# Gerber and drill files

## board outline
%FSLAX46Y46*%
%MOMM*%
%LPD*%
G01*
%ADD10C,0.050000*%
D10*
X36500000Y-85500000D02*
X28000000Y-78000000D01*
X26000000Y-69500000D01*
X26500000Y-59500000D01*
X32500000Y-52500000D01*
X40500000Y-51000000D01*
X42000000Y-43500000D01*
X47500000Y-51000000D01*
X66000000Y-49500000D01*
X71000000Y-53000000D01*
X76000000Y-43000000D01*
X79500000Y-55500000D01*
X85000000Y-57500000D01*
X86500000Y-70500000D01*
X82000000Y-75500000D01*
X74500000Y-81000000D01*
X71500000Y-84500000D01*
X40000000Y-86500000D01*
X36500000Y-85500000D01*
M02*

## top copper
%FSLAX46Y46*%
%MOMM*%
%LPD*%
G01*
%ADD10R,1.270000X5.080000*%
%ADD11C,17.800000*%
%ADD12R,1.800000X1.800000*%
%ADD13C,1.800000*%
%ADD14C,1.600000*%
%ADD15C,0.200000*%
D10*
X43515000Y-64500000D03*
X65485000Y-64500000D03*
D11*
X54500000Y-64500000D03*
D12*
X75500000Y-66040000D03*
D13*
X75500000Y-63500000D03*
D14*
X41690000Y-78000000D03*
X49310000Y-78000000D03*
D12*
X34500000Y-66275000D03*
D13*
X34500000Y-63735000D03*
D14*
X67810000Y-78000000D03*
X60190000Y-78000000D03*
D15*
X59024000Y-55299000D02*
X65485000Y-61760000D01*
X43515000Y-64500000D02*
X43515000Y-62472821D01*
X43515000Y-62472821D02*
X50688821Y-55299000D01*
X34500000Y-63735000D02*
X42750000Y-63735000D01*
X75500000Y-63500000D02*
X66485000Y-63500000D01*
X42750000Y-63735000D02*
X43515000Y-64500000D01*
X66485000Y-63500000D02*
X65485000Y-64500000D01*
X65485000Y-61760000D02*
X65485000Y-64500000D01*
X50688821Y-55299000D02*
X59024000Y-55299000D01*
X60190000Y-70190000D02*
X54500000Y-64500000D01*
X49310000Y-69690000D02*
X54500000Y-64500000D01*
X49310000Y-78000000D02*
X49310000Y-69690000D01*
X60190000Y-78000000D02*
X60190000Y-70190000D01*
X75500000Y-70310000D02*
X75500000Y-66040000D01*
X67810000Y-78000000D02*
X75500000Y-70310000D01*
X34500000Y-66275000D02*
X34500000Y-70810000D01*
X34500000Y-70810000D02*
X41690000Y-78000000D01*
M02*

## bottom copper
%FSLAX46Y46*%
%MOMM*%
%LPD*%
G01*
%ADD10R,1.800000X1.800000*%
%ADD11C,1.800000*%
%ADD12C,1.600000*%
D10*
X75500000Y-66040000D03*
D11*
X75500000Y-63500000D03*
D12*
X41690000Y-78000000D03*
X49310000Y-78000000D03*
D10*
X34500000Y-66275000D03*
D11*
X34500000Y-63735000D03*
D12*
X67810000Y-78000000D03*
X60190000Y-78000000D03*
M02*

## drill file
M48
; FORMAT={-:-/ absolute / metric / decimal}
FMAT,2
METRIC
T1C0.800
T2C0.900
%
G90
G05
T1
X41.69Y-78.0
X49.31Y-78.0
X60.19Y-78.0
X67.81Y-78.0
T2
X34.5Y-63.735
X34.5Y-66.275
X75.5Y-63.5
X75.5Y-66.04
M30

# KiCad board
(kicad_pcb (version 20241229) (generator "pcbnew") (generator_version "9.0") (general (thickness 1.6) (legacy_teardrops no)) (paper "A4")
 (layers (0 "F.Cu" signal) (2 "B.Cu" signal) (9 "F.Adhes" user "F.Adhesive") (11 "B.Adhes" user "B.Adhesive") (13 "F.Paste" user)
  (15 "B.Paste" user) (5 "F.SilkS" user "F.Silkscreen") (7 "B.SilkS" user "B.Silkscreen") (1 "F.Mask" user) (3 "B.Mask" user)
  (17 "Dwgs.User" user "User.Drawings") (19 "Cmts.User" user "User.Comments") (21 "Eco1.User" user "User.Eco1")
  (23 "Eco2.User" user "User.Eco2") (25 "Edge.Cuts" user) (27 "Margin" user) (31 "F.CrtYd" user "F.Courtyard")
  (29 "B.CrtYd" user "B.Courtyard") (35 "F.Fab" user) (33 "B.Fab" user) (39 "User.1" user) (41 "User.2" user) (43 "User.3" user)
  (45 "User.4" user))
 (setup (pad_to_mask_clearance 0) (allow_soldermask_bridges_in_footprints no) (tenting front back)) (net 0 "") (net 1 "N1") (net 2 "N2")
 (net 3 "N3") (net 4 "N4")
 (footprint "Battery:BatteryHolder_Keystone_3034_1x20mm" (layer "F.Cu") (at 54.5 64.5)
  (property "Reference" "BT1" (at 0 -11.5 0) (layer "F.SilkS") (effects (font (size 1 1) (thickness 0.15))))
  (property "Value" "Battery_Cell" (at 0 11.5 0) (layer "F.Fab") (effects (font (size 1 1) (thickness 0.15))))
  (pad "1" smd rect (at -10.985 0) (size 1.27 5.08) (layers "F.Cu" "F.Mask" "F.Paste") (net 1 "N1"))
  (pad "1" smd rect (at 10.985 0) (size 1.27 5.08) (layers "F.Cu" "F.Mask" "F.Paste") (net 1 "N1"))
  (pad "2" smd circle (at 0 0) (size 17.8 17.8) (layers "F.Cu" "F.Mask") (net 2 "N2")))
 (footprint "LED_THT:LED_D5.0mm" (layer "F.Cu") (at 75.5 66.04 90)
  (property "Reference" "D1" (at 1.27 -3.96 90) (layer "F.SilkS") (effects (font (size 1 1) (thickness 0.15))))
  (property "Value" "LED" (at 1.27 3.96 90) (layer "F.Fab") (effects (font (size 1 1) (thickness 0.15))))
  (pad "1" thru_hole rect (at 0 0 90) (size 1.8 1.8) (drill 0.9) (layers "*.Cu" "*.Mask") (remove_unused_layers no) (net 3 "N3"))
  (pad "2" thru_hole circle (at 2.54 0 90) (size 1.8 1.8) (drill 0.9) (layers "*.Cu" "*.Mask") (remove_unused_layers no) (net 1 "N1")))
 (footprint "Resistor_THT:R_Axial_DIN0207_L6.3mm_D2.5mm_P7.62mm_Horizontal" (layer "F.Cu") (at 41.69 78)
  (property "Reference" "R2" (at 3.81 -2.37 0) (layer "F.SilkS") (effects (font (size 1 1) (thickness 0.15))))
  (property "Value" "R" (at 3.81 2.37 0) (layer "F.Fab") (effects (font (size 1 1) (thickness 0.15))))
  (pad "1" thru_hole circle (at 0 0) (size 1.6 1.6) (drill 0.8) (layers "*.Cu" "*.Mask") (remove_unused_layers no) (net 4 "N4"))
  (pad "2" thru_hole circle (at 7.62 0) (size 1.6 1.6) (drill 0.8) (layers "*.Cu" "*.Mask") (remove_unused_layers no) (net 2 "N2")))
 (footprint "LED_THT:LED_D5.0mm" (layer "F.Cu") (at 34.5 66.275 90)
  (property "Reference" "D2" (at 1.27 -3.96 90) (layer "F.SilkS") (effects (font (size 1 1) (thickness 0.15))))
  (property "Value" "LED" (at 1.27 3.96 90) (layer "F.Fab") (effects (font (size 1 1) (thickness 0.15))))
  (pad "1" thru_hole rect (at 0 0 90) (size 1.8 1.8) (drill 0.9) (layers "*.Cu" "*.Mask") (remove_unused_layers no) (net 4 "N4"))
  (pad "2" thru_hole circle (at 2.54 0 90) (size 1.8 1.8) (drill 0.9) (layers "*.Cu" "*.Mask") (remove_unused_layers no) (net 1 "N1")))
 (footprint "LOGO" (layer "F.Cu") (at 72 58)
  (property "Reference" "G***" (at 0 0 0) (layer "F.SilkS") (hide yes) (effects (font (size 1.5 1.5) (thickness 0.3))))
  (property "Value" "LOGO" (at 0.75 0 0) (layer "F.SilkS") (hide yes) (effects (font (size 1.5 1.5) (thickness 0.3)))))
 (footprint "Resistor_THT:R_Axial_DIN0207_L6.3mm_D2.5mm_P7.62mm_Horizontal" (layer "F.Cu") (at 67.81 78 180)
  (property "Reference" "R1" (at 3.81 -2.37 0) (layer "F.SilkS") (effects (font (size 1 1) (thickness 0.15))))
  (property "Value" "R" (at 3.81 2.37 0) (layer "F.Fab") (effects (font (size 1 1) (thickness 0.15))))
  (pad "1" thru_hole circle (at 0 0 180) (size 1.6 1.6) (drill 0.8) (layers "*.Cu" "*.Mask") (remove_unused_layers no) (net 3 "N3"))
  (pad "2" thru_hole circle (at 7.62 0 180) (size 1.6 1.6) (drill 0.8) (layers "*.Cu" "*.Mask") (remove_unused_layers no) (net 2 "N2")))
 (gr_poly
  (pts (xy 36.5 85.5) (xy 28 78) (xy 26 69.5) (xy 26.5 59.5) (xy 32.5 52.5) (xy 40.5 51) (xy 42 43.5) (xy 47.5 51) (xy 66 49.5) (xy 71 53)
   (xy 76 43) (xy 79.5 55.5) (xy 85 57.5) (xy 86.5 70.5) (xy 82 75.5) (xy 74.5 81) (xy 71.5 84.5) (xy 40 86.5))
  (stroke (width 0.05) (type solid)) (fill no) (layer "Edge.Cuts"))
 (segment (start 59.024 55.299) (end 65.485 61.76) (width 0.2) (layer "F.Cu") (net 1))
 (segment (start 43.515 64.5) (end 43.515 62.472821) (width 0.2) (layer "F.Cu") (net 1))
 (segment (start 43.515 62.472821) (end 50.688821 55.299) (width 0.2) (layer "F.Cu") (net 1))
 (segment (start 34.5 63.735) (end 42.75 63.735) (width 0.2) (layer "F.Cu") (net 1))
 (segment (start 75.5 63.5) (end 66.485 63.5) (width 0.2) (layer "F.Cu") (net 1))
 (segment (start 42.75 63.735) (end 43.515 64.5) (width 0.2) (layer "F.Cu") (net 1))
 (segment (start 66.485 63.5) (end 65.485 64.5) (width 0.2) (layer "F.Cu") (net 1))
 (segment (start 65.485 61.76) (end 65.485 64.5) (width 0.2) (layer "F.Cu") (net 1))
 (segment (start 50.688821 55.299) (end 59.024 55.299) (width 0.2) (layer "F.Cu") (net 1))
 (segment (start 60.19 70.19) (end 54.5 64.5) (width 0.2) (layer "F.Cu") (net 2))
 (segment (start 49.31 69.69) (end 54.5 64.5) (width 0.2) (layer "F.Cu") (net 2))
 (segment (start 49.31 78) (end 49.31 69.69) (width 0.2) (layer "F.Cu") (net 2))
 (segment (start 60.19 78) (end 60.19 70.19) (width 0.2) (layer "F.Cu") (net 2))
 (segment (start 75.5 70.31) (end 75.5 66.04) (width 0.2) (layer "F.Cu") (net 3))
 (segment (start 67.81 78) (end 75.5 70.31) (width 0.2) (layer "F.Cu") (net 3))
 (segment (start 34.5 66.275) (end 34.5 70.81) (width 0.2) (layer "F.Cu") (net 4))
 (segment (start 34.5 70.81) (end 41.69 78) (width 0.2) (layer "F.Cu") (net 4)))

